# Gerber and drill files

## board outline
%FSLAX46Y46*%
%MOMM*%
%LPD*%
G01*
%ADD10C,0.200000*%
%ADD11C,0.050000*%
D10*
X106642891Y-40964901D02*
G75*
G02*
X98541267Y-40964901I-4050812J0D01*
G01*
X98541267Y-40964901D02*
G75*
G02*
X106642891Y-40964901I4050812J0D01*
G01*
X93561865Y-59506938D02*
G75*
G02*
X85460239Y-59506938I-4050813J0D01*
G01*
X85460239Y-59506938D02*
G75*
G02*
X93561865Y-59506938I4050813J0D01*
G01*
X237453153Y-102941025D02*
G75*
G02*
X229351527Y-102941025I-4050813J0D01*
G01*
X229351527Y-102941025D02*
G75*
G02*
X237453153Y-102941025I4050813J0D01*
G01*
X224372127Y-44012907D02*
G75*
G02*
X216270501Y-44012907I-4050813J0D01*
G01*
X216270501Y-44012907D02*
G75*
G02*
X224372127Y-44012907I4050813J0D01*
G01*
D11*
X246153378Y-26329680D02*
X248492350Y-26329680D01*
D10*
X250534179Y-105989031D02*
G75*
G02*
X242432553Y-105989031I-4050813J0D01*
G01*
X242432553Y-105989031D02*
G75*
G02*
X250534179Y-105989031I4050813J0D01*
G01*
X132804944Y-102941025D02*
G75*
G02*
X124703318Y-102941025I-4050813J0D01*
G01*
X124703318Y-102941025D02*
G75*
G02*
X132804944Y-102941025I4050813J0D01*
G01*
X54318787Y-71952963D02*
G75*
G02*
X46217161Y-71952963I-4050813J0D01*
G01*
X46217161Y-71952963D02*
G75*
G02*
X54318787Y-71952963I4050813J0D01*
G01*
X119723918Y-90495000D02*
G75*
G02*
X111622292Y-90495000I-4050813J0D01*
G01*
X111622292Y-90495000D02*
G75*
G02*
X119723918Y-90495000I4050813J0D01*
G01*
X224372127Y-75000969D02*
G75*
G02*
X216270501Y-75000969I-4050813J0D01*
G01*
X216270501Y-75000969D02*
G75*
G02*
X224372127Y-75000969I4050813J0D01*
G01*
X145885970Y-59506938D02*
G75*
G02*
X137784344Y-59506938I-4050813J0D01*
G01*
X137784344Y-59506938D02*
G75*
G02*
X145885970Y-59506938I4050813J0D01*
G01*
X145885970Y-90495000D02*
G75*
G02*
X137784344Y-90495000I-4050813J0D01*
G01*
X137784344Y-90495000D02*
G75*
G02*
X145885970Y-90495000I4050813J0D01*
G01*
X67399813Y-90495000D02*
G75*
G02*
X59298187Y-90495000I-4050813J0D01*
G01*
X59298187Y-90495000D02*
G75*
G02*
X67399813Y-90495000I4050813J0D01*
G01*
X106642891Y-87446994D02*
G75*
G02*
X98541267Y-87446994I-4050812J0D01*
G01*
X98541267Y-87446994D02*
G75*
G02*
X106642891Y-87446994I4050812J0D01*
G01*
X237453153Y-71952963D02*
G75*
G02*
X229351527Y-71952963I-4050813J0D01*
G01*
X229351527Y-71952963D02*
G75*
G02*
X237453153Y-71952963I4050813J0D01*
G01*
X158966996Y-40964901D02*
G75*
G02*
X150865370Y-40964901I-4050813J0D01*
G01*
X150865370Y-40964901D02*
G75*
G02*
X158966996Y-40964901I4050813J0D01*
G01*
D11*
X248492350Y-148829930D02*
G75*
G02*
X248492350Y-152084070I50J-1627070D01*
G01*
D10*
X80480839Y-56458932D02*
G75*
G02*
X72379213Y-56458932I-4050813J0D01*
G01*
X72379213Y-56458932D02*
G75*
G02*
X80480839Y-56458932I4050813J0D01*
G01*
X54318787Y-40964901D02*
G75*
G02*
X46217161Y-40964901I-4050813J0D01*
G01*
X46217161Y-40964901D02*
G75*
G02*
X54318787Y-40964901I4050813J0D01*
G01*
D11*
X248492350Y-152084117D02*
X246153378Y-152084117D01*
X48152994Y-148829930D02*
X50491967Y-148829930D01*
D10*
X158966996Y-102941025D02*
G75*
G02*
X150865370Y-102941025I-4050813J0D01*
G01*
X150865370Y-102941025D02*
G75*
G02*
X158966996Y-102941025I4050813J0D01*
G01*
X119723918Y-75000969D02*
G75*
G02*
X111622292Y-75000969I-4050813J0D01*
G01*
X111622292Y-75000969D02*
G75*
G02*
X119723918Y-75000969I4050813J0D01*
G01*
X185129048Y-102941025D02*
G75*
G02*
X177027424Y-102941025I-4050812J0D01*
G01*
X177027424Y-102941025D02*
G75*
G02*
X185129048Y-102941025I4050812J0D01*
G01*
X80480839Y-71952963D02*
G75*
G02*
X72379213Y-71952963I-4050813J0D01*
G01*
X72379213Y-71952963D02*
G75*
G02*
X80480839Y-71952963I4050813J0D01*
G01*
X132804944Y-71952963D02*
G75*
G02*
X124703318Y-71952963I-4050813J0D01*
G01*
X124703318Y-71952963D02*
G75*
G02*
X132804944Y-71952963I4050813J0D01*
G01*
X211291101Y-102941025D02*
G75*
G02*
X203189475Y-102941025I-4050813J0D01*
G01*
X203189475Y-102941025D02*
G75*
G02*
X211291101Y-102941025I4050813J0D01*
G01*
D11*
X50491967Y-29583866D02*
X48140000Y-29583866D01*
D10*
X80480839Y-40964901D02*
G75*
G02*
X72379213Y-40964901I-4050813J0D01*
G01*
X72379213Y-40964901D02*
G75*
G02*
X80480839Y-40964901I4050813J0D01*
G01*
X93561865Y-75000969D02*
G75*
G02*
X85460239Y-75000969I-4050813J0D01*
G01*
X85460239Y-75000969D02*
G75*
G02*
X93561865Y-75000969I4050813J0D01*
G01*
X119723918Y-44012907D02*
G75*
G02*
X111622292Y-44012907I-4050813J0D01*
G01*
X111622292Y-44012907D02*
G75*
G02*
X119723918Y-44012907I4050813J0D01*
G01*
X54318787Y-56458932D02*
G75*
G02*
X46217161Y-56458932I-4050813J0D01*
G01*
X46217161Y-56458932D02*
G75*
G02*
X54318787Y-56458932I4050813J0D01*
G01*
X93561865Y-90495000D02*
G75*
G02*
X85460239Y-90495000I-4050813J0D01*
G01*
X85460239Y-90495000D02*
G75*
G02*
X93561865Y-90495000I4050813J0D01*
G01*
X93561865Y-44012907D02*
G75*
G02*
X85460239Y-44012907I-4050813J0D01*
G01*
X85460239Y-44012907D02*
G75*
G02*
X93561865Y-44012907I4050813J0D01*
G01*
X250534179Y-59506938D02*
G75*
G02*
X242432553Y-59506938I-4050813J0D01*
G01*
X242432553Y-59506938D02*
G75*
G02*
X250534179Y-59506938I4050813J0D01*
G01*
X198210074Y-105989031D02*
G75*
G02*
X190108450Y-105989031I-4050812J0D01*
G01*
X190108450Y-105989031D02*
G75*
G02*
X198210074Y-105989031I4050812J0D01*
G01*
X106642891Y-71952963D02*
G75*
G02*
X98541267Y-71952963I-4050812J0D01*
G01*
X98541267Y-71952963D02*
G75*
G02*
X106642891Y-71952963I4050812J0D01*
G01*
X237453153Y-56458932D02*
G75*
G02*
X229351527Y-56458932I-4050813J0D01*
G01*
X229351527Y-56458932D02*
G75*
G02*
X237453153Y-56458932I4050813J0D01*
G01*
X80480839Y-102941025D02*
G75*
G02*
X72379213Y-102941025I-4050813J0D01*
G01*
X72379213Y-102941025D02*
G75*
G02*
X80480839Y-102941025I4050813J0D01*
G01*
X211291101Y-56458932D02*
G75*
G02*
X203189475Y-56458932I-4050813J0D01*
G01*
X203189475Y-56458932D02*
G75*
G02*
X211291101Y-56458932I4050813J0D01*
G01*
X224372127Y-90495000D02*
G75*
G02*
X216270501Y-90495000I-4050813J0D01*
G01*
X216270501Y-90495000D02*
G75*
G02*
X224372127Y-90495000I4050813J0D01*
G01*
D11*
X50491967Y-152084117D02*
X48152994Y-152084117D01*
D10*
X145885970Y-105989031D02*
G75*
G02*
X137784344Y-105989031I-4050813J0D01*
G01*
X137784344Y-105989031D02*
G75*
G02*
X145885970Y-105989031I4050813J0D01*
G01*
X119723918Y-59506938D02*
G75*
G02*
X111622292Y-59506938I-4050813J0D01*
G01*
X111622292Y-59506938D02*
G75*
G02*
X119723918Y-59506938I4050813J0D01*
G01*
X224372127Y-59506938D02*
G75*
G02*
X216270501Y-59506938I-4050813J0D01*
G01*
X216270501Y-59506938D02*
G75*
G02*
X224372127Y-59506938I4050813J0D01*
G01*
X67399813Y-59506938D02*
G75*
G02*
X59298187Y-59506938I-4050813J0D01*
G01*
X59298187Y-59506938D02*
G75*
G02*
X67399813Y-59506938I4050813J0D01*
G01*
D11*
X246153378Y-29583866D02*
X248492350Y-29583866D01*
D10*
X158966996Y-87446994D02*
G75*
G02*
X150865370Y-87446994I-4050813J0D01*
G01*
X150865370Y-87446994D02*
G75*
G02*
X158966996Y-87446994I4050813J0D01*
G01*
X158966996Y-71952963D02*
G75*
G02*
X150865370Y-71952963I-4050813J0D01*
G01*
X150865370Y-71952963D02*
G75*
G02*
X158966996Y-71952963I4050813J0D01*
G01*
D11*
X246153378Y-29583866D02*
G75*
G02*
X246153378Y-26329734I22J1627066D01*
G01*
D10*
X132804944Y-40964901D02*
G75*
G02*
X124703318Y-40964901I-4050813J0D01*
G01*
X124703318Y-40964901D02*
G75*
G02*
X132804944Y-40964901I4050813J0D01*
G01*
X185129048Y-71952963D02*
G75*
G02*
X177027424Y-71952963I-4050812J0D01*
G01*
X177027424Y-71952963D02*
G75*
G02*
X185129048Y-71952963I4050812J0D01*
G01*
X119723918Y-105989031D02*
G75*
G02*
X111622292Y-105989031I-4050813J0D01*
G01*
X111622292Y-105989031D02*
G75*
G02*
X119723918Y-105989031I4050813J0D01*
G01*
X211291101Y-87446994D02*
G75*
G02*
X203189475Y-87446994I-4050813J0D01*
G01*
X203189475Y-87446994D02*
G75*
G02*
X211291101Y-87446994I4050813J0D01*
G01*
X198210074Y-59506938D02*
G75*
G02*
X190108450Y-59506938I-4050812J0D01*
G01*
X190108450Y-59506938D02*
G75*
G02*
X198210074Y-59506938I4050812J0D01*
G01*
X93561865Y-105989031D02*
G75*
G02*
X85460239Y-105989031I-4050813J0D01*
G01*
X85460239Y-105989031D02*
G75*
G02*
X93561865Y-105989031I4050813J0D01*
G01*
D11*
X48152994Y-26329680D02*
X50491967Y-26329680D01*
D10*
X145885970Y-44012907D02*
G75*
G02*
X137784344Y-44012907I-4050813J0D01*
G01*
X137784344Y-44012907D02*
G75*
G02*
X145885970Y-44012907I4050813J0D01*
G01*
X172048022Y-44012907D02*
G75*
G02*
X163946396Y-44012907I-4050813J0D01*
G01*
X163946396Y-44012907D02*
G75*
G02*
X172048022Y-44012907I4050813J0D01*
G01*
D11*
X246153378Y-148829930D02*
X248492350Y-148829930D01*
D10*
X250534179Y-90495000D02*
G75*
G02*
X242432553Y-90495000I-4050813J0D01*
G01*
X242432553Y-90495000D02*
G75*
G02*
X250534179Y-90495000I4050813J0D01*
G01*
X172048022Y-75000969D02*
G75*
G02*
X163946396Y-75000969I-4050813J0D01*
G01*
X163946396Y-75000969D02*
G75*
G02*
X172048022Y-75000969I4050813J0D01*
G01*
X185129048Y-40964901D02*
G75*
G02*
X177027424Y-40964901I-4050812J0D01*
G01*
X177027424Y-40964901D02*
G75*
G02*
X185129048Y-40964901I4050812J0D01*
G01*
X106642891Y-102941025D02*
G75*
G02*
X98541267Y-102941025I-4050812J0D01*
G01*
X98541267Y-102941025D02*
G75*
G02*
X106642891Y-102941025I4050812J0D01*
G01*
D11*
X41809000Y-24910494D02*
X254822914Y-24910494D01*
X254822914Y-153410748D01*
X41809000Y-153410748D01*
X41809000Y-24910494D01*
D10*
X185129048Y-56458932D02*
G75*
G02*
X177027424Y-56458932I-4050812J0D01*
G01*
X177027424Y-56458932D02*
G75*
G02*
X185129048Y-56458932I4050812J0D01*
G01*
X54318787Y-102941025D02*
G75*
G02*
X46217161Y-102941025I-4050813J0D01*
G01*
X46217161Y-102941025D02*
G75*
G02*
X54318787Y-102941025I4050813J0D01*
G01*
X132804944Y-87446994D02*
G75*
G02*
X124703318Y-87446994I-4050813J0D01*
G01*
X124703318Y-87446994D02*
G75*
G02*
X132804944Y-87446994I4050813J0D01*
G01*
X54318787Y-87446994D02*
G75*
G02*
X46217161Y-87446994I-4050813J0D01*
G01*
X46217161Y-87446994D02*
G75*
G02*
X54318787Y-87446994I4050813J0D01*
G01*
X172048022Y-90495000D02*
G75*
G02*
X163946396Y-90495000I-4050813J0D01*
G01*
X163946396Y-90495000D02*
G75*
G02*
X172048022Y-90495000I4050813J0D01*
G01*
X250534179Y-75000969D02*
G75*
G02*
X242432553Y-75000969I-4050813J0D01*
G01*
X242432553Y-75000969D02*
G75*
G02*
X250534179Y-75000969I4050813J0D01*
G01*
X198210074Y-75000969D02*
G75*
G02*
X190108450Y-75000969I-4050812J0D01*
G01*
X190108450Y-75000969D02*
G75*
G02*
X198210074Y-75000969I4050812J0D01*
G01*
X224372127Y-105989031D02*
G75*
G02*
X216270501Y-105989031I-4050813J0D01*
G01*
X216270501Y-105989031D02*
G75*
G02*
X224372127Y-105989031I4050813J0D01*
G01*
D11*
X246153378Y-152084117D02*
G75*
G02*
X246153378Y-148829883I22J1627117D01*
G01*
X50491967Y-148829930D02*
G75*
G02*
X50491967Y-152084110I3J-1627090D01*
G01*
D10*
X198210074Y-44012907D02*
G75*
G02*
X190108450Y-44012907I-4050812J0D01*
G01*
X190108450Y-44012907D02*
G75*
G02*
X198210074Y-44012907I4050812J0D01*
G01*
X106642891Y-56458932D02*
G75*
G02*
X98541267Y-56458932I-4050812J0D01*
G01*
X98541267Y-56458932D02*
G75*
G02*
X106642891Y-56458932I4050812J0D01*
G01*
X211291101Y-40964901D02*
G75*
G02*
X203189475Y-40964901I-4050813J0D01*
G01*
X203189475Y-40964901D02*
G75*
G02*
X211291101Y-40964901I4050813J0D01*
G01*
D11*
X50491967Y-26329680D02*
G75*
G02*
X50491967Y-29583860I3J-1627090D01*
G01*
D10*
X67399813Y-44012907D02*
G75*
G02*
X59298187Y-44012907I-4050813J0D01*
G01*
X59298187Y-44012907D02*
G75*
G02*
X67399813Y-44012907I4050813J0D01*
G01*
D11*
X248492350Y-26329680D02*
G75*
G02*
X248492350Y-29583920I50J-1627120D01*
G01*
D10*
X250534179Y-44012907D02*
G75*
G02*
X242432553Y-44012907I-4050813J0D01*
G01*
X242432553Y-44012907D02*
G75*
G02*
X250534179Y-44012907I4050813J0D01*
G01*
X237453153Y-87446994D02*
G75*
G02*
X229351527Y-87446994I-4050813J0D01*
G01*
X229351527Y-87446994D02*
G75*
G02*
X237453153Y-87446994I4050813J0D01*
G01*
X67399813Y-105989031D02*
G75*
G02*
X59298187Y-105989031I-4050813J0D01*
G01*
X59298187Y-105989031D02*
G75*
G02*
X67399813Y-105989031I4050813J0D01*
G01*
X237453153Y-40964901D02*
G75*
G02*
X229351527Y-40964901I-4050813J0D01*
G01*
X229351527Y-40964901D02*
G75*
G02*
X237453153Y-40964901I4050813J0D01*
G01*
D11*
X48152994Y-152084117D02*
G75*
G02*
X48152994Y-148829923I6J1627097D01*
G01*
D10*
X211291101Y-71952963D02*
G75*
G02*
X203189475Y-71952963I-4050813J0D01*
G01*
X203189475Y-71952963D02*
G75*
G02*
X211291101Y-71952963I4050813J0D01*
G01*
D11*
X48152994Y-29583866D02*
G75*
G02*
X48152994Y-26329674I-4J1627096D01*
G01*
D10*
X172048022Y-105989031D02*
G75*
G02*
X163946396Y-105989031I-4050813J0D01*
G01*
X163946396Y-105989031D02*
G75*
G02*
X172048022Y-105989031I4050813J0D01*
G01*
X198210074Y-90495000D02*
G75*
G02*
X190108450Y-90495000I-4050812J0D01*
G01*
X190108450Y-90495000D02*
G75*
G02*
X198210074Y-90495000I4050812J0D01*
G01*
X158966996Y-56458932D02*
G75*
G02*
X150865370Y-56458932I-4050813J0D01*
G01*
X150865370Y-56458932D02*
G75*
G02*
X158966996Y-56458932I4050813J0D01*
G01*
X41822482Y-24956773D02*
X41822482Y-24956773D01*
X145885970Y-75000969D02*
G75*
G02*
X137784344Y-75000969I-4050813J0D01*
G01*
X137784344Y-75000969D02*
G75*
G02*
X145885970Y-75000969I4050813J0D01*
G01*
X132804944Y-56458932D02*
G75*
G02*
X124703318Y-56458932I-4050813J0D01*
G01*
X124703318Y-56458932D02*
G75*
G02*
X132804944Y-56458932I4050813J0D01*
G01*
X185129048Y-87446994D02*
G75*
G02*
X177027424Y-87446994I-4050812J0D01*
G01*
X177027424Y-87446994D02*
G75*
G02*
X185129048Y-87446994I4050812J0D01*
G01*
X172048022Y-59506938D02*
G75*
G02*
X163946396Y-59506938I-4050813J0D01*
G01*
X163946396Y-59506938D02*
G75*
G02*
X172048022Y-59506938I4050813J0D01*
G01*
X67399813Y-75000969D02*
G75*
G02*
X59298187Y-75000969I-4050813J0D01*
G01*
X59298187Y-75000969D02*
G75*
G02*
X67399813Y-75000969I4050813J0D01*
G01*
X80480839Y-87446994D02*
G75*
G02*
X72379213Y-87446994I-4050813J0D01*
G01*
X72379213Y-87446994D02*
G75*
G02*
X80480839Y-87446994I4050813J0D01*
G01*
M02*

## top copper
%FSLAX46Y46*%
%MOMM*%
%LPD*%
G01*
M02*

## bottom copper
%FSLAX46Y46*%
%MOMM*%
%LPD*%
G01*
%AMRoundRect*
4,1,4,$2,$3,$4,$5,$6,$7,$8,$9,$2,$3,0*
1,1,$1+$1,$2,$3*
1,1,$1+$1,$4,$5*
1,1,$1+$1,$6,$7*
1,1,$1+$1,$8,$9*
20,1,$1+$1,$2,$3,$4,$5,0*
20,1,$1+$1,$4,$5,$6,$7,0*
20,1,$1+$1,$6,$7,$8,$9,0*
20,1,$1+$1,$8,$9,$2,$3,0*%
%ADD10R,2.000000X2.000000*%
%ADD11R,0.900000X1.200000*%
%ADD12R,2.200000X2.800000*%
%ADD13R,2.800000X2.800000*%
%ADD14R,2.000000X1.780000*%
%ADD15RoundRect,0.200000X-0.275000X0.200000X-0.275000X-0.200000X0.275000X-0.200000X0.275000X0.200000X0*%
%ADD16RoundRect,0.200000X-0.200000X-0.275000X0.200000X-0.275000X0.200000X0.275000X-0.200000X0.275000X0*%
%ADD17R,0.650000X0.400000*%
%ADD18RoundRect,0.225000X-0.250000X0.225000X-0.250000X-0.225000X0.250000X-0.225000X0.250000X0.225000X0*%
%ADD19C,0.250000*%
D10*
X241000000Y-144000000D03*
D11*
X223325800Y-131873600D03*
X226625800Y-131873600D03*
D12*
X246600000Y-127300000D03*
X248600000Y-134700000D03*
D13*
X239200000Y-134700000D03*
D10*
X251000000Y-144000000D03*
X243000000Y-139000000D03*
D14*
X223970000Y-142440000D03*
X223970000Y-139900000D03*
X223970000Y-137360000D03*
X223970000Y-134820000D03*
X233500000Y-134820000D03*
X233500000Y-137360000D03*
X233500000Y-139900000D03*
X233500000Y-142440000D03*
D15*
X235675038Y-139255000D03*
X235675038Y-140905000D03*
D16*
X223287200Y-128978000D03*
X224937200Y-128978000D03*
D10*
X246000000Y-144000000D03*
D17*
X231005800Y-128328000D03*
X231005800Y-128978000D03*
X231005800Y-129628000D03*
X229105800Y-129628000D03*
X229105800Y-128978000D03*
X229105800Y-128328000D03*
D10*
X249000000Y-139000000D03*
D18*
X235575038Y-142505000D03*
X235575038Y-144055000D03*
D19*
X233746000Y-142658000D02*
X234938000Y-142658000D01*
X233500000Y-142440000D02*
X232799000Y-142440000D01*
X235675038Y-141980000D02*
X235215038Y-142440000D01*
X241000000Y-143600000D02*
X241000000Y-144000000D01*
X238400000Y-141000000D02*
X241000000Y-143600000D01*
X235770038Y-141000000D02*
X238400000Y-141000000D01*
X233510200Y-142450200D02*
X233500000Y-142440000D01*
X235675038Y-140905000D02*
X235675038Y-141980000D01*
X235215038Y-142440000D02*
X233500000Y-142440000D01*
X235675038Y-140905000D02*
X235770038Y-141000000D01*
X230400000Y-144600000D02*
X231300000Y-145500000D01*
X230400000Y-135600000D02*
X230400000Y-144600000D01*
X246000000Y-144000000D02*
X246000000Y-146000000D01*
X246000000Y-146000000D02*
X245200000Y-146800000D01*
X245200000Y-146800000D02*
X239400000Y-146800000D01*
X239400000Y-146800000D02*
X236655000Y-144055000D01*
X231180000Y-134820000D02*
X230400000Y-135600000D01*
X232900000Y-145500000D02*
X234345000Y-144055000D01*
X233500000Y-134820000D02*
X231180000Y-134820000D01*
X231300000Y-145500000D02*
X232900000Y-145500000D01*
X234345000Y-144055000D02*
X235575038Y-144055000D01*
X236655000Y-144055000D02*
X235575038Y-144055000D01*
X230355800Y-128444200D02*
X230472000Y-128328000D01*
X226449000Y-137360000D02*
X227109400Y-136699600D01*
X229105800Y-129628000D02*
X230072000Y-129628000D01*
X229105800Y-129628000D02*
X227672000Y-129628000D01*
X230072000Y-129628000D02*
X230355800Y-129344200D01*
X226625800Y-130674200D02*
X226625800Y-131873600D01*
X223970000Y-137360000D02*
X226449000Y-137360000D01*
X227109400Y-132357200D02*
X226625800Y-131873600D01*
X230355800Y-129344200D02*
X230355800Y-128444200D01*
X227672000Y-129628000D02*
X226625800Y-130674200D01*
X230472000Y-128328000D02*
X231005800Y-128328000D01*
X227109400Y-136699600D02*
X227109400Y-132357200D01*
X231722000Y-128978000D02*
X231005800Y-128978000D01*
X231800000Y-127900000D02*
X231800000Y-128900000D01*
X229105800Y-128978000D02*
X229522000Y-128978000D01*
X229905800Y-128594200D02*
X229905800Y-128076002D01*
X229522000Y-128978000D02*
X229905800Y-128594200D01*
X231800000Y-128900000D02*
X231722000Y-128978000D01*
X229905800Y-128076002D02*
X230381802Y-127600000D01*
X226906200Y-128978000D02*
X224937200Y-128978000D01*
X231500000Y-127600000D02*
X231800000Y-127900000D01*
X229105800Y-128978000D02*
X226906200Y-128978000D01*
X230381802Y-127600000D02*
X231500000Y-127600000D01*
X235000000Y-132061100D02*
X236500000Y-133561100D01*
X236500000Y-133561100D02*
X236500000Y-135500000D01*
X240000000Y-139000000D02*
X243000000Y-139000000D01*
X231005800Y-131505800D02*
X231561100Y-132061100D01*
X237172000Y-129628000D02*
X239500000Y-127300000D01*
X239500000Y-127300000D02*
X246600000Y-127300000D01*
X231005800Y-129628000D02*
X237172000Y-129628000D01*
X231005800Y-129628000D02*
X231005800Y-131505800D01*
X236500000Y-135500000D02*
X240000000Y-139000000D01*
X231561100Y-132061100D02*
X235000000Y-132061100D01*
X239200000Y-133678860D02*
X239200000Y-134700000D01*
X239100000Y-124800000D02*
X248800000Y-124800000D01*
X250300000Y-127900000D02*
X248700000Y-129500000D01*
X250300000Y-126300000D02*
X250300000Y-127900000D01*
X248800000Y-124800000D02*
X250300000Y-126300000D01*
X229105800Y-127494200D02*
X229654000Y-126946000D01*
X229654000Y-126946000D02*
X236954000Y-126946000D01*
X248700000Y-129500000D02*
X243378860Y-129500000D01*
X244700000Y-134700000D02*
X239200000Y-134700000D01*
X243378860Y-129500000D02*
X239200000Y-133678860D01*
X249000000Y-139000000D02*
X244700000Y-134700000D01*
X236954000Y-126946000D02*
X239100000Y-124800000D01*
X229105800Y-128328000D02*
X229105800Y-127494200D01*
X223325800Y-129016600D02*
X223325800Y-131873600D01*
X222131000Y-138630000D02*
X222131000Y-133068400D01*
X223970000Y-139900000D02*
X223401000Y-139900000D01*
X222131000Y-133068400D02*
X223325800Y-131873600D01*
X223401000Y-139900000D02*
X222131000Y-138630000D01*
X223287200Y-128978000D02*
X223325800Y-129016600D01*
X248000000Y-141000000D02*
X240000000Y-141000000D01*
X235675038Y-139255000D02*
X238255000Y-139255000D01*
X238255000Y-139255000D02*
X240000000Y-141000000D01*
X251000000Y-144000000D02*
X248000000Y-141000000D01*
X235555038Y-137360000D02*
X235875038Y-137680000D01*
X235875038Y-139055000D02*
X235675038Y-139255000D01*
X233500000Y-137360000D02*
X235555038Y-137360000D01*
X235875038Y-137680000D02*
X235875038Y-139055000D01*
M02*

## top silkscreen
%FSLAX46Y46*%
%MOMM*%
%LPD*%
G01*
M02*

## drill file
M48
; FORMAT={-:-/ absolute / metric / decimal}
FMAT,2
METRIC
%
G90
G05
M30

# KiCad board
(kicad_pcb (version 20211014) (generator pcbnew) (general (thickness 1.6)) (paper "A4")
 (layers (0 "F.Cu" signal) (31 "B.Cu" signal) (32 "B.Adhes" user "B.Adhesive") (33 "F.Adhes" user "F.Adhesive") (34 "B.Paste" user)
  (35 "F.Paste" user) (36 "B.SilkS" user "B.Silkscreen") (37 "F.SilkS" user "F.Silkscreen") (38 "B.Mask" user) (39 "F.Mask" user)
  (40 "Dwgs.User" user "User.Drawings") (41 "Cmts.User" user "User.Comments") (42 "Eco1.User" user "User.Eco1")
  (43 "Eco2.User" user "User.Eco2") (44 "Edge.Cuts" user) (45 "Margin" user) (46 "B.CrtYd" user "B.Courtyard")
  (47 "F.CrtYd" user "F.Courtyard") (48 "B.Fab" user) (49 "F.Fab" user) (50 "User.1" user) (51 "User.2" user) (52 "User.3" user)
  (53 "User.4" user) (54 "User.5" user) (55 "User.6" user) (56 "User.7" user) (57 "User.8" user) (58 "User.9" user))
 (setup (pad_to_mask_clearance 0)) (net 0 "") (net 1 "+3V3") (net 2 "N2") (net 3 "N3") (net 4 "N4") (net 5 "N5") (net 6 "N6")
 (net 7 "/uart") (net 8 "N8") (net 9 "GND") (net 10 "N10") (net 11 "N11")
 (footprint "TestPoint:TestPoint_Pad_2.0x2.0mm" (layer "B.Cu") (at 241 144 180)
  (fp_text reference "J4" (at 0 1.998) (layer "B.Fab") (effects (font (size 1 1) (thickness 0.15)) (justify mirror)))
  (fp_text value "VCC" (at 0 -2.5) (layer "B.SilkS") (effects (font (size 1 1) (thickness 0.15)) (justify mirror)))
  (pad "1" smd rect (at 0 0 180) (size 2 2) (layers "B.Cu" "B.Mask") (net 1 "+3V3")))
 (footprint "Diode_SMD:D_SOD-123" (layer "B.Cu") (at 224.9758 131.8736)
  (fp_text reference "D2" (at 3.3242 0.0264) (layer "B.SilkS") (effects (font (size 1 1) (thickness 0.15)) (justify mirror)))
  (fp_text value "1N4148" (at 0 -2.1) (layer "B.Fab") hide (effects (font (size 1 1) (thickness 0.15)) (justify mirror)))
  (pad "1" smd rect (at -1.65 0) (size 0.9 1.2) (layers "B.Cu" "B.Paste" "B.Mask") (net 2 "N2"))
  (pad "2" smd rect (at 1.65 0) (size 0.9 1.2) (layers "B.Cu" "B.Paste" "B.Mask") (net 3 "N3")))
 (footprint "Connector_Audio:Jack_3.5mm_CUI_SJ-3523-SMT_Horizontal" (layer "B.Cu") (at 245 131 90)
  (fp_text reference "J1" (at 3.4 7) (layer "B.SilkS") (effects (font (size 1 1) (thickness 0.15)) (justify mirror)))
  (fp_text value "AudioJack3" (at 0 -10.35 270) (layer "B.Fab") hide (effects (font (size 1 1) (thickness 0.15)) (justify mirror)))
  (pad "R" smd rect (at 3.7 1.6 90) (size 2.8 2.2) (layers "B.Cu" "B.Paste" "B.Mask") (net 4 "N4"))
  (pad "S" smd rect (at -3.7 3.6 90) (size 2.8 2.2) (layers "B.Cu" "B.Paste" "B.Mask") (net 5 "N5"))
  (pad "T" smd rect (at -3.7 -5.8 90) (size 2.8 2.8) (layers "B.Cu" "B.Paste" "B.Mask") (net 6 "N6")))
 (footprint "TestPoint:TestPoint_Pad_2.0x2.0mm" (layer "B.Cu") (at 251 144 180)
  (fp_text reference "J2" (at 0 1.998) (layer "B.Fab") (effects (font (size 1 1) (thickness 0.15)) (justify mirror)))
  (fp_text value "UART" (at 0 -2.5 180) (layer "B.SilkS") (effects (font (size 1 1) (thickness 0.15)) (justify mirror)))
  (pad "1" smd rect (at 0 0 180) (size 2 2) (layers "B.Cu" "B.Mask") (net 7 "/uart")))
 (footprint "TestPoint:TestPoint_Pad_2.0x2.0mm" (layer "B.Cu") (at 243 139 180)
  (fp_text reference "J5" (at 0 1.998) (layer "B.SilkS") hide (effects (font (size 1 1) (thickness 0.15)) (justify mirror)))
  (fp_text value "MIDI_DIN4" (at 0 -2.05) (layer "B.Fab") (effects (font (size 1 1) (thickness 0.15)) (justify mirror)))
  (pad "1" smd rect (at 0 0 180) (size 2 2) (layers "B.Cu" "B.Mask") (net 4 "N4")))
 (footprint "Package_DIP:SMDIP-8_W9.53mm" (layer "B.Cu") (at 228.735 138.63)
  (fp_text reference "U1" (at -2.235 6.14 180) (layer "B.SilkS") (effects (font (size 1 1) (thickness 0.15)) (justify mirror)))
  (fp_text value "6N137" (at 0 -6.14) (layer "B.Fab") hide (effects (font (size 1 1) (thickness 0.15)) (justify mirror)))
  (pad "1" smd rect (at -4.765 3.81) (size 2 1.78) (layers "B.Cu" "B.Paste" "B.Mask") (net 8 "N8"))
  (pad "2" smd rect (at -4.765 1.27) (size 2 1.78) (layers "B.Cu" "B.Paste" "B.Mask") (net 2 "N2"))
  (pad "3" smd rect (at -4.765 -1.27) (size 2 1.78) (layers "B.Cu" "B.Paste" "B.Mask") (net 3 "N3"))
  (pad "4" smd rect (at -4.765 -3.81) (size 2 1.78) (layers "B.Cu" "B.Paste" "B.Mask"))
  (pad "5" smd rect (at 4.765 -3.81) (size 2 1.78) (layers "B.Cu" "B.Paste" "B.Mask") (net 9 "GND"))
  (pad "6" smd rect (at 4.765 -1.27) (size 2 1.78) (layers "B.Cu" "B.Paste" "B.Mask") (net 7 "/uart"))
  (pad "7" smd rect (at 4.765 1.27) (size 2 1.78) (layers "B.Cu" "B.Paste" "B.Mask") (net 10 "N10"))
  (pad "8" smd rect (at 4.765 3.81) (size 2 1.78) (layers "B.Cu" "B.Paste" "B.Mask") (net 1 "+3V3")))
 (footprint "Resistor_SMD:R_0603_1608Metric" (layer "B.Cu") (at 235.675038 140.08 -90)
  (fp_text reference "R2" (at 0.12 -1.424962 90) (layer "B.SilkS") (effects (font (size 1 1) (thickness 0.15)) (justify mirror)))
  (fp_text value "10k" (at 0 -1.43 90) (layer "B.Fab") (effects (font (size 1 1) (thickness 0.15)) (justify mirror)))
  (pad "1" smd roundrect (at -0.825 0 270) (size 0.8 0.95) (layers "B.Cu" "B.Paste" "B.Mask") (roundrect_rratio 0.25) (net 7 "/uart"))
  (pad "2" smd roundrect (at 0.825 0 270) (size 0.8 0.95) (layers "B.Cu" "B.Paste" "B.Mask") (roundrect_rratio 0.25) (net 1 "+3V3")))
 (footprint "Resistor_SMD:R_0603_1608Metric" (layer "B.Cu") (at 224.1122 128.978)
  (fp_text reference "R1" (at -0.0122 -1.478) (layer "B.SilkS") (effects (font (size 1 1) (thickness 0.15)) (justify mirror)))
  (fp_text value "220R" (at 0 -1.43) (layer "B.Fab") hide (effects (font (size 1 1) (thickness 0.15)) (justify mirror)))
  (pad "1" smd roundrect (at -0.825 0) (size 0.8 0.95) (layers "B.Cu" "B.Paste" "B.Mask") (roundrect_rratio 0.25) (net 2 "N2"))
  (pad "2" smd roundrect (at 0.825 0) (size 0.8 0.95) (layers "B.Cu" "B.Paste" "B.Mask") (roundrect_rratio 0.25) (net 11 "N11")))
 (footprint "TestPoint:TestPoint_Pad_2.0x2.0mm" (layer "B.Cu") (at 246 144 180)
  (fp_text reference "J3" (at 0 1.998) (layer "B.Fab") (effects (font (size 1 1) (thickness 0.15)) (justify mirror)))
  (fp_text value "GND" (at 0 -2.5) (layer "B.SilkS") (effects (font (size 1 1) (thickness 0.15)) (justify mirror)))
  (pad "1" smd rect (at 0 0 180) (size 2 2) (layers "B.Cu" "B.Mask") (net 9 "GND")))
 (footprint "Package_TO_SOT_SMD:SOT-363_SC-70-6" (layer "B.Cu") (at 230.0558 128.978 180)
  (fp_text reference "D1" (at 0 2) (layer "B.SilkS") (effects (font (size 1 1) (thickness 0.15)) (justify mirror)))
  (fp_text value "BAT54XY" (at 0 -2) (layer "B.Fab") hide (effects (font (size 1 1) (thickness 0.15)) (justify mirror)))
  (pad "1" smd rect (at -0.95 0.65 180) (size 0.65 0.4) (layers "B.Cu" "B.Paste" "B.Mask") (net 3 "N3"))
  (pad "2" smd rect (at -0.95 0 180) (size 0.65 0.4) (layers "B.Cu" "B.Paste" "B.Mask") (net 11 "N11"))
  (pad "3" smd rect (at -0.95 -0.65 180) (size 0.65 0.4) (layers "B.Cu" "B.Paste" "B.Mask") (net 4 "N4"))
  (pad "4" smd rect (at 0.95 -0.65 180) (size 0.65 0.4) (layers "B.Cu" "B.Paste" "B.Mask") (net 3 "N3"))
  (pad "5" smd rect (at 0.95 0 180) (size 0.65 0.4) (layers "B.Cu" "B.Paste" "B.Mask") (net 11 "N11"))
  (pad "6" smd rect (at 0.95 0.65 180) (size 0.65 0.4) (layers "B.Cu" "B.Paste" "B.Mask") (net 6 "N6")))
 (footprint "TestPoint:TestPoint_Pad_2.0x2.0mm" (layer "B.Cu") (at 249 139 180)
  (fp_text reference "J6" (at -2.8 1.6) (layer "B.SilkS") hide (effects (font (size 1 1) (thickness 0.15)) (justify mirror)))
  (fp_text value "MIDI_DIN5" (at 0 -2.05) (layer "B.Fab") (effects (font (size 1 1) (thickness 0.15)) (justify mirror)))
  (pad "1" smd rect (at 0 0 180) (size 2 2) (layers "B.Cu" "B.Mask") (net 6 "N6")))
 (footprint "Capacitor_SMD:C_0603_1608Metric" (layer "B.Cu") (at 235.575038 143.28 -90)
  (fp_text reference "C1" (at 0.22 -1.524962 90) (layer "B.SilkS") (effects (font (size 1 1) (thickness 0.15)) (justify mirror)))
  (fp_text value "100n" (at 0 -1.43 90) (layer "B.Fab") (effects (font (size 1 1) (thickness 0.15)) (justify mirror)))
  (pad "1" smd roundrect (at -0.775 0 270) (size 0.9 0.95) (layers "B.Cu" "B.Paste" "B.Mask") (roundrect_rratio 0.25) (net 1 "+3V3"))
  (pad "2" smd roundrect (at 0.775 0 270) (size 0.9 0.95) (layers "B.Cu" "B.Paste" "B.Mask") (roundrect_rratio 0.25) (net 9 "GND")))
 (gr_circle (center 102.592079 40.964901) (end 106.642891 40.964901) (layer "Edge.Cuts") (width 0.2) (fill none))
 (gr_circle (center 89.511052 59.506938) (end 93.561865 59.506938) (layer "Edge.Cuts") (width 0.2) (fill none))
 (gr_circle (center 233.40234 102.941025) (end 237.453153 102.941025) (layer "Edge.Cuts") (width 0.2) (fill none))
 (gr_circle (center 220.321314 44.012907) (end 224.372127 44.012907) (layer "Edge.Cuts") (width 0.2) (fill none))
 (gr_line (start 246.153378 26.32968) (end 248.49235 26.32968) (layer "Edge.Cuts") (width 0.05))
 (gr_circle (center 246.483366 105.989031) (end 250.534179 105.989031) (layer "Edge.Cuts") (width 0.2) (fill none))
 (gr_circle (center 128.754131 102.941025) (end 132.804944 102.941025) (layer "Edge.Cuts") (width 0.2) (fill none))
 (gr_circle (center 50.267974 71.952963) (end 54.318787 71.952963) (layer "Edge.Cuts") (width 0.2) (fill none))
 (gr_circle (center 115.673105 90.495) (end 119.723918 90.495) (layer "Edge.Cuts") (width 0.2) (fill none))
 (gr_circle (center 220.321314 75.000969) (end 224.372127 75.000969) (layer "Edge.Cuts") (width 0.2) (fill none))
 (gr_circle (center 141.835157 59.506938) (end 145.88597 59.506938) (layer "Edge.Cuts") (width 0.2) (fill none))
 (gr_circle (center 141.835157 90.495) (end 145.88597 90.495) (layer "Edge.Cuts") (width 0.2) (fill none))
 (gr_circle (center 63.349 90.495) (end 67.399813 90.495) (layer "Edge.Cuts") (width 0.2) (fill none))
 (gr_circle (center 102.592079 87.446994) (end 106.642891 87.446994) (layer "Edge.Cuts") (width 0.2) (fill none))
 (gr_circle (center 233.40234 71.952963) (end 237.453153 71.952963) (layer "Edge.Cuts") (width 0.2) (fill none))
 (gr_circle (center 154.916183 40.964901) (end 158.966996 40.964901) (layer "Edge.Cuts") (width 0.2) (fill none))
 (gr_arc (start 248.49235 148.82993) (mid 250.119451 150.457024) (end 248.49235 152.084117) (layer "Edge.Cuts") (width 0.05))
 (gr_circle (center 76.430026 56.458932) (end 80.480839 56.458932) (layer "Edge.Cuts") (width 0.2) (fill none))
 (gr_circle (center 50.267974 40.964901) (end 54.318787 40.964901) (layer "Edge.Cuts") (width 0.2) (fill none))
 (gr_line (start 248.49235 152.084117) (end 246.153378 152.084117) (layer "Edge.Cuts") (width 0.05))
 (gr_line (start 48.152994 148.82993) (end 50.491967 148.82993) (layer "Edge.Cuts") (width 0.05))
 (gr_circle (center 154.916183 102.941025) (end 158.966996 102.941025) (layer "Edge.Cuts") (width 0.2) (fill none))
 (gr_circle (center 115.673105 75.000969) (end 119.723918 75.000969) (layer "Edge.Cuts") (width 0.2) (fill none))
 (gr_circle (center 181.078236 102.941025) (end 185.129048 102.941025) (layer "Edge.Cuts") (width 0.2) (fill none))
 (gr_circle (center 76.430026 71.952963) (end 80.480839 71.952963) (layer "Edge.Cuts") (width 0.2) (fill none))
 (gr_circle (center 128.754131 71.952963) (end 132.804944 71.952963) (layer "Edge.Cuts") (width 0.2) (fill none))
 (gr_circle (center 207.240288 102.941025) (end 211.291101 102.941025) (layer "Edge.Cuts") (width 0.2) (fill none))
 (gr_line (start 50.491967 29.583866) (end 48.14 29.583866) (layer "Edge.Cuts") (width 0.05))
 (gr_circle (center 76.430026 40.964901) (end 80.480839 40.964901) (layer "Edge.Cuts") (width 0.2) (fill none))
 (gr_circle (center 89.511052 75.000969) (end 93.561865 75.000969) (layer "Edge.Cuts") (width 0.2) (fill none))
 (gr_circle (center 115.673105 44.012907) (end 119.723918 44.012907) (layer "Edge.Cuts") (width 0.2) (fill none))
 (gr_circle (center 50.267974 56.458932) (end 54.318787 56.458932) (layer "Edge.Cuts") (width 0.2) (fill none))
 (gr_circle (center 89.511052 90.495) (end 93.561865 90.495) (layer "Edge.Cuts") (width 0.2) (fill none))
 (gr_circle (center 89.511052 44.012907) (end 93.561865 44.012907) (layer "Edge.Cuts") (width 0.2) (fill none))
 (gr_circle (center 246.483366 59.506938) (end 250.534179 59.506938) (layer "Edge.Cuts") (width 0.2) (fill none))
 (gr_circle (center 194.159262 105.989031) (end 198.210074 105.989031) (layer "Edge.Cuts") (width 0.2) (fill none))
 (gr_circle (center 102.592079 71.952963) (end 106.642891 71.952963) (layer "Edge.Cuts") (width 0.2) (fill none))
 (gr_circle (center 233.40234 56.458932) (end 237.453153 56.458932) (layer "Edge.Cuts") (width 0.2) (fill none))
 (gr_circle (center 76.430026 102.941025) (end 80.480839 102.941025) (layer "Edge.Cuts") (width 0.2) (fill none))
 (gr_circle (center 207.240288 56.458932) (end 211.291101 56.458932) (layer "Edge.Cuts") (width 0.2) (fill none))
 (gr_circle (center 220.321314 90.495) (end 224.372127 90.495) (layer "Edge.Cuts") (width 0.2) (fill none))
 (gr_line (start 50.491967 152.084117) (end 48.152994 152.084117) (layer "Edge.Cuts") (width 0.05))
 (gr_circle (center 141.835157 105.989031) (end 145.88597 105.989031) (layer "Edge.Cuts") (width 0.2) (fill none))
 (gr_circle (center 115.673105 59.506938) (end 119.723918 59.506938) (layer "Edge.Cuts") (width 0.2) (fill none))
 (gr_circle (center 220.321314 59.506938) (end 224.372127 59.506938) (layer "Edge.Cuts") (width 0.2) (fill none))
 (gr_circle (center 63.349 59.506938) (end 67.399813 59.506938) (layer "Edge.Cuts") (width 0.2) (fill none))
 (gr_line (start 246.153378 29.583866) (end 248.49235 29.583866) (layer "Edge.Cuts") (width 0.05))
 (gr_circle (center 154.916183 87.446994) (end 158.966996 87.446994) (layer "Edge.Cuts") (width 0.2) (fill none))
 (gr_circle (center 154.916183 71.952963) (end 158.966996 71.952963) (layer "Edge.Cuts") (width 0.2) (fill none))
 (gr_arc (start 246.153378 29.583866) (mid 244.526264 27.956773) (end 246.153378 26.32968) (layer "Edge.Cuts") (width 0.05))
 (gr_circle (center 128.754131 40.964901) (end 132.804944 40.964901) (layer "Edge.Cuts") (width 0.2) (fill none))
 (gr_circle (center 181.078236 71.952963) (end 185.129048 71.952963) (layer "Edge.Cuts") (width 0.2) (fill none))
 (gr_circle (center 115.673105 105.989031) (end 119.723918 105.989031) (layer "Edge.Cuts") (width 0.2) (fill none))
 (gr_circle (center 207.240288 87.446994) (end 211.291101 87.446994) (layer "Edge.Cuts") (width 0.2) (fill none))
 (gr_circle (center 194.159262 59.506938) (end 198.210074 59.506938) (layer "Edge.Cuts") (width 0.2) (fill none))
 (gr_circle (center 89.511052 105.989031) (end 93.561865 105.989031) (layer "Edge.Cuts") (width 0.2) (fill none))
 (gr_line (start 48.152994 26.32968) (end 50.491967 26.32968) (layer "Edge.Cuts") (width 0.05))
 (gr_circle (center 141.835157 44.012907) (end 145.88597 44.012907) (layer "Edge.Cuts") (width 0.2) (fill none))
 (gr_circle (center 167.997209 44.012907) (end 172.048022 44.012907) (layer "Edge.Cuts") (width 0.2) (fill none))
 (gr_line (start 246.153378 148.82993) (end 248.49235 148.82993) (layer "Edge.Cuts") (width 0.05))
 (gr_circle (center 246.483366 90.495) (end 250.534179 90.495) (layer "Edge.Cuts") (width 0.2) (fill none))
 (gr_circle (center 167.997209 75.000969) (end 172.048022 75.000969) (layer "Edge.Cuts") (width 0.2) (fill none))
 (gr_circle (center 181.078236 40.964901) (end 185.129048 40.964901) (layer "Edge.Cuts") (width 0.2) (fill none))
 (gr_circle (center 102.592079 102.941025) (end 106.642891 102.941025) (layer "Edge.Cuts") (width 0.2) (fill none))
 (gr_rect (start 254.822914 24.910494) (end 41.809 153.410748) (layer "Edge.Cuts") (width 0.05) (fill none))
 (gr_circle (center 181.078236 56.458932) (end 185.129048 56.458932) (layer "Edge.Cuts") (width 0.2) (fill none))
 (gr_circle (center 50.267974 102.941025) (end 54.318787 102.941025) (layer "Edge.Cuts") (width 0.2) (fill none))
 (gr_circle (center 128.754131 87.446994) (end 132.804944 87.446994) (layer "Edge.Cuts") (width 0.2) (fill none))
 (gr_circle (center 50.267974 87.446994) (end 54.318787 87.446994) (layer "Edge.Cuts") (width 0.2) (fill none))
 (gr_circle (center 167.997209 90.495) (end 172.048022 90.495) (layer "Edge.Cuts") (width 0.2) (fill none))
 (gr_circle (center 246.483366 75.000969) (end 250.534179 75.000969) (layer "Edge.Cuts") (width 0.2) (fill none))
 (gr_circle (center 194.159262 75.000969) (end 198.210074 75.000969) (layer "Edge.Cuts") (width 0.2) (fill none))
 (gr_circle (center 220.321314 105.989031) (end 224.372127 105.989031) (layer "Edge.Cuts") (width 0.2) (fill none))
 (gr_arc (start 246.153378 152.084117) (mid 244.526264 150.457024) (end 246.153378 148.82993) (layer "Edge.Cuts") (width 0.05))
 (gr_arc (start 50.491967 148.82993) (mid 52.119061 150.457024) (end 50.491967 152.084117) (layer "Edge.Cuts") (width 0.05))
 (gr_circle (center 194.159262 44.012907) (end 198.210074 44.012907) (layer "Edge.Cuts") (width 0.2) (fill none))
 (gr_circle (center 102.592079 56.458932) (end 106.642891 56.458932) (layer "Edge.Cuts") (width 0.2) (fill none))
 (gr_circle (center 207.240288 40.964901) (end 211.291101 40.964901) (layer "Edge.Cuts") (width 0.2) (fill none))
 (gr_arc (start 50.491967 26.32968) (mid 52.11906 27.956773) (end 50.491967 29.583866) (layer "Edge.Cuts") (width 0.05))
 (gr_circle (center 63.349 44.012907) (end 67.399813 44.012907) (layer "Edge.Cuts") (width 0.2) (fill none))
 (gr_arc (start 248.49235 26.32968) (mid 250.11945 27.956773) (end 248.49235 29.583866) (layer "Edge.Cuts") (width 0.05))
 (gr_circle (center 246.483366 44.012907) (end 250.534179 44.012907) (layer "Edge.Cuts") (width 0.2) (fill none))
 (gr_circle (center 233.40234 87.446994) (end 237.453153 87.446994) (layer "Edge.Cuts") (width 0.2) (fill none))
 (gr_circle (center 63.349 105.989031) (end 67.399813 105.989031) (layer "Edge.Cuts") (width 0.2) (fill none))
 (gr_circle (center 233.40234 40.964901) (end 237.453153 40.964901) (layer "Edge.Cuts") (width 0.2) (fill none))
 (gr_arc (start 48.152994 152.084117) (mid 46.525904 150.457024) (end 48.152994 148.82993) (layer "Edge.Cuts") (width 0.05))
 (gr_circle (center 207.240288 71.952963) (end 211.291101 71.952963) (layer "Edge.Cuts") (width 0.2) (fill none))
 (gr_arc (start 48.152994 29.583866) (mid 46.525901 27.956773) (end 48.152994 26.32968) (layer "Edge.Cuts") (width 0.05))
 (gr_circle (center 167.997209 105.989031) (end 172.048022 105.989031) (layer "Edge.Cuts") (width 0.2) (fill none))
 (gr_circle (center 194.159262 90.495) (end 198.210074 90.495) (layer "Edge.Cuts") (width 0.2) (fill none))
 (gr_circle (center 154.916183 56.458932) (end 158.966996 56.458932) (layer "Edge.Cuts") (width 0.2) (fill none))
 (gr_line (start 41.822482 24.956773) (end 41.822482 24.956773) (layer "Edge.Cuts") (width 0.2))
 (gr_circle (center 141.835157 75.000969) (end 145.88597 75.000969) (layer "Edge.Cuts") (width 0.2) (fill none))
 (gr_circle (center 128.754131 56.458932) (end 132.804944 56.458932) (layer "Edge.Cuts") (width 0.2) (fill none))
 (gr_circle (center 181.078236 87.446994) (end 185.129048 87.446994) (layer "Edge.Cuts") (width 0.2) (fill none))
 (gr_circle (center 167.997209 59.506938) (end 172.048022 59.506938) (layer "Edge.Cuts") (width 0.2) (fill none))
 (gr_circle (center 63.349 75.000969) (end 67.399813 75.000969) (layer "Edge.Cuts") (width 0.2) (fill none))
 (gr_circle (center 76.430026 87.446994) (end 80.480839 87.446994) (layer "Edge.Cuts") (width 0.2) (fill none))
 (segment (start 233.746 142.658) (end 234.938 142.658) (width 0.25) (layer "B.Cu") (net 1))
 (segment (start 233.5 142.44) (end 232.799 142.44) (width 0.25) (layer "B.Cu") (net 1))
 (segment (start 235.675038 141.98) (end 235.215038 142.44) (width 0.25) (layer "B.Cu") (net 1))
 (segment (start 241 143.6) (end 241 144) (width 0.25) (layer "B.Cu") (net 1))
 (segment (start 238.4 141) (end 241 143.6) (width 0.25) (layer "B.Cu") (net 1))
 (segment (start 235.770038 141) (end 238.4 141) (width 0.25) (layer "B.Cu") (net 1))
 (segment (start 233.5102 142.4502) (end 233.5 142.44) (width 0.25) (layer "B.Cu") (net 1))
 (segment (start 235.675038 140.905) (end 235.675038 141.98) (width 0.25) (layer "B.Cu") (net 1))
 (segment (start 235.215038 142.44) (end 233.5 142.44) (width 0.25) (layer "B.Cu") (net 1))
 (segment (start 235.675038 140.905) (end 235.770038 141) (width 0.25) (layer "B.Cu") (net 1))
 (segment (start 230.4 144.6) (end 231.3 145.5) (width 0.25) (layer "B.Cu") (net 9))
 (segment (start 230.4 135.6) (end 230.4 144.6) (width 0.25) (layer "B.Cu") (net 9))
 (segment (start 246 144) (end 246 146) (width 0.25) (layer "B.Cu") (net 9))
 (segment (start 246 146) (end 245.2 146.8) (width 0.25) (layer "B.Cu") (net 9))
 (segment (start 245.2 146.8) (end 239.4 146.8) (width 0.25) (layer "B.Cu") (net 9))
 (segment (start 239.4 146.8) (end 236.655 144.055) (width 0.25) (layer "B.Cu") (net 9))
 (segment (start 231.18 134.82) (end 230.4 135.6) (width 0.25) (layer "B.Cu") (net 9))
 (segment (start 232.9 145.5) (end 234.345 144.055) (width 0.25) (layer "B.Cu") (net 9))
 (segment (start 233.5 134.82) (end 231.18 134.82) (width 0.25) (layer "B.Cu") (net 9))
 (segment (start 231.3 145.5) (end 232.9 145.5) (width 0.25) (layer "B.Cu") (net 9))
 (segment (start 234.345 144.055) (end 235.575038 144.055) (width 0.25) (layer "B.Cu") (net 9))
 (segment (start 236.655 144.055) (end 235.575038 144.055) (width 0.25) (layer "B.Cu") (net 9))
 (segment (start 230.3558 128.4442) (end 230.472 128.328) (width 0.25) (layer "B.Cu") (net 3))
 (segment (start 226.449 137.36) (end 227.1094 136.6996) (width 0.25) (layer "B.Cu") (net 3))
 (segment (start 229.1058 129.628) (end 230.072 129.628) (width 0.25) (layer "B.Cu") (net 3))
 (segment (start 229.1058 129.628) (end 227.672 129.628) (width 0.25) (layer "B.Cu") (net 3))
 (segment (start 230.072 129.628) (end 230.3558 129.3442) (width 0.25) (layer "B.Cu") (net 3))
 (segment (start 226.6258 130.6742) (end 226.6258 131.8736) (width 0.25) (layer "B.Cu") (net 3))
 (segment (start 223.97 137.36) (end 226.449 137.36) (width 0.25) (layer "B.Cu") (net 3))
 (segment (start 227.1094 132.3572) (end 226.6258 131.8736) (width 0.25) (layer "B.Cu") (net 3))
 (segment (start 230.3558 129.3442) (end 230.3558 128.4442) (width 0.25) (layer "B.Cu") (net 3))
 (segment (start 227.672 129.628) (end 226.6258 130.6742) (width 0.25) (layer "B.Cu") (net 3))
 (segment (start 230.472 128.328) (end 231.0058 128.328) (width 0.25) (layer "B.Cu") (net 3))
 (segment (start 227.1094 136.6996) (end 227.1094 132.3572) (width 0.25) (layer "B.Cu") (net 3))
 (segment (start 231.722 128.978) (end 231.0058 128.978) (width 0.25) (layer "B.Cu") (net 11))
 (segment (start 231.8 127.9) (end 231.8 128.9) (width 0.25) (layer "B.Cu") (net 11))
 (segment (start 229.1058 128.978) (end 229.522 128.978) (width 0.25) (layer "B.Cu") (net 11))
 (segment (start 229.9058 128.5942) (end 229.9058 128.076002) (width 0.25) (layer "B.Cu") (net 11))
 (segment (start 229.522 128.978) (end 229.9058 128.5942) (width 0.25) (layer "B.Cu") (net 11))
 (segment (start 231.8 128.9) (end 231.722 128.978) (width 0.25) (layer "B.Cu") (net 11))
 (segment (start 229.9058 128.076002) (end 230.381802 127.6) (width 0.25) (layer "B.Cu") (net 11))
 (segment (start 226.9062 128.978) (end 224.9372 128.978) (width 0.25) (layer "B.Cu") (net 11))
 (segment (start 231.5 127.6) (end 231.8 127.9) (width 0.25) (layer "B.Cu") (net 11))
 (segment (start 229.1058 128.978) (end 226.9062 128.978) (width 0.25) (layer "B.Cu") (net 11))
 (segment (start 230.381802 127.6) (end 231.5 127.6) (width 0.25) (layer "B.Cu") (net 11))
 (segment (start 235 132.0611) (end 236.5 133.5611) (width 0.25) (layer "B.Cu") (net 4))
 (segment (start 236.5 133.5611) (end 236.5 135.5) (width 0.25) (layer "B.Cu") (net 4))
 (segment (start 240 139) (end 243 139) (width 0.25) (layer "B.Cu") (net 4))
 (segment (start 231.0058 131.5058) (end 231.5611 132.0611) (width 0.25) (layer "B.Cu") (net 4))
 (segment (start 237.172 129.628) (end 239.5 127.3) (width 0.25) (layer "B.Cu") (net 4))
 (segment (start 239.5 127.3) (end 246.6 127.3) (width 0.25) (layer "B.Cu") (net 4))
 (segment (start 231.0058 129.628) (end 237.172 129.628) (width 0.25) (layer "B.Cu") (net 4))
 (segment (start 231.0058 129.628) (end 231.0058 131.5058) (width 0.25) (layer "B.Cu") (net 4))
 (segment (start 236.5 135.5) (end 240 139) (width 0.25) (layer "B.Cu") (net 4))
 (segment (start 231.5611 132.0611) (end 235 132.0611) (width 0.25) (layer "B.Cu") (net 4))
 (segment (start 239.2 133.67886) (end 239.2 134.7) (width 0.25) (layer "B.Cu") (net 6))
 (segment (start 239.1 124.8) (end 248.8 124.8) (width 0.25) (layer "B.Cu") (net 6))
 (segment (start 250.3 127.9) (end 248.7 129.5) (width 0.25) (layer "B.Cu") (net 6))
 (segment (start 250.3 126.3) (end 250.3 127.9) (width 0.25) (layer "B.Cu") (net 6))
 (segment (start 248.8 124.8) (end 250.3 126.3) (width 0.25) (layer "B.Cu") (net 6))
 (segment (start 229.1058 127.4942) (end 229.654 126.946) (width 0.25) (layer "B.Cu") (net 6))
 (segment (start 229.654 126.946) (end 236.954 126.946) (width 0.25) (layer "B.Cu") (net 6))
 (segment (start 248.7 129.5) (end 243.37886 129.5) (width 0.25) (layer "B.Cu") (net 6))
 (segment (start 244.7 134.7) (end 239.2 134.7) (width 0.25) (layer "B.Cu") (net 6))
 (segment (start 243.37886 129.5) (end 239.2 133.67886) (width 0.25) (layer "B.Cu") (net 6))
 (segment (start 249 139) (end 244.7 134.7) (width 0.25) (layer "B.Cu") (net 6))
 (segment (start 236.954 126.946) (end 239.1 124.8) (width 0.25) (layer "B.Cu") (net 6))
 (segment (start 229.1058 128.328) (end 229.1058 127.4942) (width 0.25) (layer "B.Cu") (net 6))
 (segment (start 223.3258 129.0166) (end 223.3258 131.8736) (width 0.25) (layer "B.Cu") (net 2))
 (segment (start 222.131 138.63) (end 222.131 133.0684) (width 0.25) (layer "B.Cu") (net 2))
 (segment (start 223.97 139.9) (end 223.401 139.9) (width 0.25) (layer "B.Cu") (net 2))
 (segment (start 222.131 133.0684) (end 223.3258 131.8736) (width 0.25) (layer "B.Cu") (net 2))
 (segment (start 223.401 139.9) (end 222.131 138.63) (width 0.25) (layer "B.Cu") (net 2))
 (segment (start 223.2872 128.978) (end 223.3258 129.0166) (width 0.25) (layer "B.Cu") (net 2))
 (segment (start 248 141) (end 240 141) (width 0.25) (layer "B.Cu") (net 7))
 (segment (start 235.675038 139.255) (end 238.255 139.255) (width 0.25) (layer "B.Cu") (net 7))
 (segment (start 238.255 139.255) (end 240 141) (width 0.25) (layer "B.Cu") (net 7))
 (segment (start 251 144) (end 248 141) (width 0.25) (layer "B.Cu") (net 7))
 (segment (start 235.555038 137.36) (end 235.875038 137.68) (width 0.25) (layer "B.Cu") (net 7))
 (segment (start 235.875038 139.055) (end 235.675038 139.255) (width 0.25) (layer "B.Cu") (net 7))
 (segment (start 233.5 137.36) (end 235.555038 137.36) (width 0.25) (layer "B.Cu") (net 7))
 (segment (start 235.875038 137.68) (end 235.875038 139.055) (width 0.25) (layer "B.Cu") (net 7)))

